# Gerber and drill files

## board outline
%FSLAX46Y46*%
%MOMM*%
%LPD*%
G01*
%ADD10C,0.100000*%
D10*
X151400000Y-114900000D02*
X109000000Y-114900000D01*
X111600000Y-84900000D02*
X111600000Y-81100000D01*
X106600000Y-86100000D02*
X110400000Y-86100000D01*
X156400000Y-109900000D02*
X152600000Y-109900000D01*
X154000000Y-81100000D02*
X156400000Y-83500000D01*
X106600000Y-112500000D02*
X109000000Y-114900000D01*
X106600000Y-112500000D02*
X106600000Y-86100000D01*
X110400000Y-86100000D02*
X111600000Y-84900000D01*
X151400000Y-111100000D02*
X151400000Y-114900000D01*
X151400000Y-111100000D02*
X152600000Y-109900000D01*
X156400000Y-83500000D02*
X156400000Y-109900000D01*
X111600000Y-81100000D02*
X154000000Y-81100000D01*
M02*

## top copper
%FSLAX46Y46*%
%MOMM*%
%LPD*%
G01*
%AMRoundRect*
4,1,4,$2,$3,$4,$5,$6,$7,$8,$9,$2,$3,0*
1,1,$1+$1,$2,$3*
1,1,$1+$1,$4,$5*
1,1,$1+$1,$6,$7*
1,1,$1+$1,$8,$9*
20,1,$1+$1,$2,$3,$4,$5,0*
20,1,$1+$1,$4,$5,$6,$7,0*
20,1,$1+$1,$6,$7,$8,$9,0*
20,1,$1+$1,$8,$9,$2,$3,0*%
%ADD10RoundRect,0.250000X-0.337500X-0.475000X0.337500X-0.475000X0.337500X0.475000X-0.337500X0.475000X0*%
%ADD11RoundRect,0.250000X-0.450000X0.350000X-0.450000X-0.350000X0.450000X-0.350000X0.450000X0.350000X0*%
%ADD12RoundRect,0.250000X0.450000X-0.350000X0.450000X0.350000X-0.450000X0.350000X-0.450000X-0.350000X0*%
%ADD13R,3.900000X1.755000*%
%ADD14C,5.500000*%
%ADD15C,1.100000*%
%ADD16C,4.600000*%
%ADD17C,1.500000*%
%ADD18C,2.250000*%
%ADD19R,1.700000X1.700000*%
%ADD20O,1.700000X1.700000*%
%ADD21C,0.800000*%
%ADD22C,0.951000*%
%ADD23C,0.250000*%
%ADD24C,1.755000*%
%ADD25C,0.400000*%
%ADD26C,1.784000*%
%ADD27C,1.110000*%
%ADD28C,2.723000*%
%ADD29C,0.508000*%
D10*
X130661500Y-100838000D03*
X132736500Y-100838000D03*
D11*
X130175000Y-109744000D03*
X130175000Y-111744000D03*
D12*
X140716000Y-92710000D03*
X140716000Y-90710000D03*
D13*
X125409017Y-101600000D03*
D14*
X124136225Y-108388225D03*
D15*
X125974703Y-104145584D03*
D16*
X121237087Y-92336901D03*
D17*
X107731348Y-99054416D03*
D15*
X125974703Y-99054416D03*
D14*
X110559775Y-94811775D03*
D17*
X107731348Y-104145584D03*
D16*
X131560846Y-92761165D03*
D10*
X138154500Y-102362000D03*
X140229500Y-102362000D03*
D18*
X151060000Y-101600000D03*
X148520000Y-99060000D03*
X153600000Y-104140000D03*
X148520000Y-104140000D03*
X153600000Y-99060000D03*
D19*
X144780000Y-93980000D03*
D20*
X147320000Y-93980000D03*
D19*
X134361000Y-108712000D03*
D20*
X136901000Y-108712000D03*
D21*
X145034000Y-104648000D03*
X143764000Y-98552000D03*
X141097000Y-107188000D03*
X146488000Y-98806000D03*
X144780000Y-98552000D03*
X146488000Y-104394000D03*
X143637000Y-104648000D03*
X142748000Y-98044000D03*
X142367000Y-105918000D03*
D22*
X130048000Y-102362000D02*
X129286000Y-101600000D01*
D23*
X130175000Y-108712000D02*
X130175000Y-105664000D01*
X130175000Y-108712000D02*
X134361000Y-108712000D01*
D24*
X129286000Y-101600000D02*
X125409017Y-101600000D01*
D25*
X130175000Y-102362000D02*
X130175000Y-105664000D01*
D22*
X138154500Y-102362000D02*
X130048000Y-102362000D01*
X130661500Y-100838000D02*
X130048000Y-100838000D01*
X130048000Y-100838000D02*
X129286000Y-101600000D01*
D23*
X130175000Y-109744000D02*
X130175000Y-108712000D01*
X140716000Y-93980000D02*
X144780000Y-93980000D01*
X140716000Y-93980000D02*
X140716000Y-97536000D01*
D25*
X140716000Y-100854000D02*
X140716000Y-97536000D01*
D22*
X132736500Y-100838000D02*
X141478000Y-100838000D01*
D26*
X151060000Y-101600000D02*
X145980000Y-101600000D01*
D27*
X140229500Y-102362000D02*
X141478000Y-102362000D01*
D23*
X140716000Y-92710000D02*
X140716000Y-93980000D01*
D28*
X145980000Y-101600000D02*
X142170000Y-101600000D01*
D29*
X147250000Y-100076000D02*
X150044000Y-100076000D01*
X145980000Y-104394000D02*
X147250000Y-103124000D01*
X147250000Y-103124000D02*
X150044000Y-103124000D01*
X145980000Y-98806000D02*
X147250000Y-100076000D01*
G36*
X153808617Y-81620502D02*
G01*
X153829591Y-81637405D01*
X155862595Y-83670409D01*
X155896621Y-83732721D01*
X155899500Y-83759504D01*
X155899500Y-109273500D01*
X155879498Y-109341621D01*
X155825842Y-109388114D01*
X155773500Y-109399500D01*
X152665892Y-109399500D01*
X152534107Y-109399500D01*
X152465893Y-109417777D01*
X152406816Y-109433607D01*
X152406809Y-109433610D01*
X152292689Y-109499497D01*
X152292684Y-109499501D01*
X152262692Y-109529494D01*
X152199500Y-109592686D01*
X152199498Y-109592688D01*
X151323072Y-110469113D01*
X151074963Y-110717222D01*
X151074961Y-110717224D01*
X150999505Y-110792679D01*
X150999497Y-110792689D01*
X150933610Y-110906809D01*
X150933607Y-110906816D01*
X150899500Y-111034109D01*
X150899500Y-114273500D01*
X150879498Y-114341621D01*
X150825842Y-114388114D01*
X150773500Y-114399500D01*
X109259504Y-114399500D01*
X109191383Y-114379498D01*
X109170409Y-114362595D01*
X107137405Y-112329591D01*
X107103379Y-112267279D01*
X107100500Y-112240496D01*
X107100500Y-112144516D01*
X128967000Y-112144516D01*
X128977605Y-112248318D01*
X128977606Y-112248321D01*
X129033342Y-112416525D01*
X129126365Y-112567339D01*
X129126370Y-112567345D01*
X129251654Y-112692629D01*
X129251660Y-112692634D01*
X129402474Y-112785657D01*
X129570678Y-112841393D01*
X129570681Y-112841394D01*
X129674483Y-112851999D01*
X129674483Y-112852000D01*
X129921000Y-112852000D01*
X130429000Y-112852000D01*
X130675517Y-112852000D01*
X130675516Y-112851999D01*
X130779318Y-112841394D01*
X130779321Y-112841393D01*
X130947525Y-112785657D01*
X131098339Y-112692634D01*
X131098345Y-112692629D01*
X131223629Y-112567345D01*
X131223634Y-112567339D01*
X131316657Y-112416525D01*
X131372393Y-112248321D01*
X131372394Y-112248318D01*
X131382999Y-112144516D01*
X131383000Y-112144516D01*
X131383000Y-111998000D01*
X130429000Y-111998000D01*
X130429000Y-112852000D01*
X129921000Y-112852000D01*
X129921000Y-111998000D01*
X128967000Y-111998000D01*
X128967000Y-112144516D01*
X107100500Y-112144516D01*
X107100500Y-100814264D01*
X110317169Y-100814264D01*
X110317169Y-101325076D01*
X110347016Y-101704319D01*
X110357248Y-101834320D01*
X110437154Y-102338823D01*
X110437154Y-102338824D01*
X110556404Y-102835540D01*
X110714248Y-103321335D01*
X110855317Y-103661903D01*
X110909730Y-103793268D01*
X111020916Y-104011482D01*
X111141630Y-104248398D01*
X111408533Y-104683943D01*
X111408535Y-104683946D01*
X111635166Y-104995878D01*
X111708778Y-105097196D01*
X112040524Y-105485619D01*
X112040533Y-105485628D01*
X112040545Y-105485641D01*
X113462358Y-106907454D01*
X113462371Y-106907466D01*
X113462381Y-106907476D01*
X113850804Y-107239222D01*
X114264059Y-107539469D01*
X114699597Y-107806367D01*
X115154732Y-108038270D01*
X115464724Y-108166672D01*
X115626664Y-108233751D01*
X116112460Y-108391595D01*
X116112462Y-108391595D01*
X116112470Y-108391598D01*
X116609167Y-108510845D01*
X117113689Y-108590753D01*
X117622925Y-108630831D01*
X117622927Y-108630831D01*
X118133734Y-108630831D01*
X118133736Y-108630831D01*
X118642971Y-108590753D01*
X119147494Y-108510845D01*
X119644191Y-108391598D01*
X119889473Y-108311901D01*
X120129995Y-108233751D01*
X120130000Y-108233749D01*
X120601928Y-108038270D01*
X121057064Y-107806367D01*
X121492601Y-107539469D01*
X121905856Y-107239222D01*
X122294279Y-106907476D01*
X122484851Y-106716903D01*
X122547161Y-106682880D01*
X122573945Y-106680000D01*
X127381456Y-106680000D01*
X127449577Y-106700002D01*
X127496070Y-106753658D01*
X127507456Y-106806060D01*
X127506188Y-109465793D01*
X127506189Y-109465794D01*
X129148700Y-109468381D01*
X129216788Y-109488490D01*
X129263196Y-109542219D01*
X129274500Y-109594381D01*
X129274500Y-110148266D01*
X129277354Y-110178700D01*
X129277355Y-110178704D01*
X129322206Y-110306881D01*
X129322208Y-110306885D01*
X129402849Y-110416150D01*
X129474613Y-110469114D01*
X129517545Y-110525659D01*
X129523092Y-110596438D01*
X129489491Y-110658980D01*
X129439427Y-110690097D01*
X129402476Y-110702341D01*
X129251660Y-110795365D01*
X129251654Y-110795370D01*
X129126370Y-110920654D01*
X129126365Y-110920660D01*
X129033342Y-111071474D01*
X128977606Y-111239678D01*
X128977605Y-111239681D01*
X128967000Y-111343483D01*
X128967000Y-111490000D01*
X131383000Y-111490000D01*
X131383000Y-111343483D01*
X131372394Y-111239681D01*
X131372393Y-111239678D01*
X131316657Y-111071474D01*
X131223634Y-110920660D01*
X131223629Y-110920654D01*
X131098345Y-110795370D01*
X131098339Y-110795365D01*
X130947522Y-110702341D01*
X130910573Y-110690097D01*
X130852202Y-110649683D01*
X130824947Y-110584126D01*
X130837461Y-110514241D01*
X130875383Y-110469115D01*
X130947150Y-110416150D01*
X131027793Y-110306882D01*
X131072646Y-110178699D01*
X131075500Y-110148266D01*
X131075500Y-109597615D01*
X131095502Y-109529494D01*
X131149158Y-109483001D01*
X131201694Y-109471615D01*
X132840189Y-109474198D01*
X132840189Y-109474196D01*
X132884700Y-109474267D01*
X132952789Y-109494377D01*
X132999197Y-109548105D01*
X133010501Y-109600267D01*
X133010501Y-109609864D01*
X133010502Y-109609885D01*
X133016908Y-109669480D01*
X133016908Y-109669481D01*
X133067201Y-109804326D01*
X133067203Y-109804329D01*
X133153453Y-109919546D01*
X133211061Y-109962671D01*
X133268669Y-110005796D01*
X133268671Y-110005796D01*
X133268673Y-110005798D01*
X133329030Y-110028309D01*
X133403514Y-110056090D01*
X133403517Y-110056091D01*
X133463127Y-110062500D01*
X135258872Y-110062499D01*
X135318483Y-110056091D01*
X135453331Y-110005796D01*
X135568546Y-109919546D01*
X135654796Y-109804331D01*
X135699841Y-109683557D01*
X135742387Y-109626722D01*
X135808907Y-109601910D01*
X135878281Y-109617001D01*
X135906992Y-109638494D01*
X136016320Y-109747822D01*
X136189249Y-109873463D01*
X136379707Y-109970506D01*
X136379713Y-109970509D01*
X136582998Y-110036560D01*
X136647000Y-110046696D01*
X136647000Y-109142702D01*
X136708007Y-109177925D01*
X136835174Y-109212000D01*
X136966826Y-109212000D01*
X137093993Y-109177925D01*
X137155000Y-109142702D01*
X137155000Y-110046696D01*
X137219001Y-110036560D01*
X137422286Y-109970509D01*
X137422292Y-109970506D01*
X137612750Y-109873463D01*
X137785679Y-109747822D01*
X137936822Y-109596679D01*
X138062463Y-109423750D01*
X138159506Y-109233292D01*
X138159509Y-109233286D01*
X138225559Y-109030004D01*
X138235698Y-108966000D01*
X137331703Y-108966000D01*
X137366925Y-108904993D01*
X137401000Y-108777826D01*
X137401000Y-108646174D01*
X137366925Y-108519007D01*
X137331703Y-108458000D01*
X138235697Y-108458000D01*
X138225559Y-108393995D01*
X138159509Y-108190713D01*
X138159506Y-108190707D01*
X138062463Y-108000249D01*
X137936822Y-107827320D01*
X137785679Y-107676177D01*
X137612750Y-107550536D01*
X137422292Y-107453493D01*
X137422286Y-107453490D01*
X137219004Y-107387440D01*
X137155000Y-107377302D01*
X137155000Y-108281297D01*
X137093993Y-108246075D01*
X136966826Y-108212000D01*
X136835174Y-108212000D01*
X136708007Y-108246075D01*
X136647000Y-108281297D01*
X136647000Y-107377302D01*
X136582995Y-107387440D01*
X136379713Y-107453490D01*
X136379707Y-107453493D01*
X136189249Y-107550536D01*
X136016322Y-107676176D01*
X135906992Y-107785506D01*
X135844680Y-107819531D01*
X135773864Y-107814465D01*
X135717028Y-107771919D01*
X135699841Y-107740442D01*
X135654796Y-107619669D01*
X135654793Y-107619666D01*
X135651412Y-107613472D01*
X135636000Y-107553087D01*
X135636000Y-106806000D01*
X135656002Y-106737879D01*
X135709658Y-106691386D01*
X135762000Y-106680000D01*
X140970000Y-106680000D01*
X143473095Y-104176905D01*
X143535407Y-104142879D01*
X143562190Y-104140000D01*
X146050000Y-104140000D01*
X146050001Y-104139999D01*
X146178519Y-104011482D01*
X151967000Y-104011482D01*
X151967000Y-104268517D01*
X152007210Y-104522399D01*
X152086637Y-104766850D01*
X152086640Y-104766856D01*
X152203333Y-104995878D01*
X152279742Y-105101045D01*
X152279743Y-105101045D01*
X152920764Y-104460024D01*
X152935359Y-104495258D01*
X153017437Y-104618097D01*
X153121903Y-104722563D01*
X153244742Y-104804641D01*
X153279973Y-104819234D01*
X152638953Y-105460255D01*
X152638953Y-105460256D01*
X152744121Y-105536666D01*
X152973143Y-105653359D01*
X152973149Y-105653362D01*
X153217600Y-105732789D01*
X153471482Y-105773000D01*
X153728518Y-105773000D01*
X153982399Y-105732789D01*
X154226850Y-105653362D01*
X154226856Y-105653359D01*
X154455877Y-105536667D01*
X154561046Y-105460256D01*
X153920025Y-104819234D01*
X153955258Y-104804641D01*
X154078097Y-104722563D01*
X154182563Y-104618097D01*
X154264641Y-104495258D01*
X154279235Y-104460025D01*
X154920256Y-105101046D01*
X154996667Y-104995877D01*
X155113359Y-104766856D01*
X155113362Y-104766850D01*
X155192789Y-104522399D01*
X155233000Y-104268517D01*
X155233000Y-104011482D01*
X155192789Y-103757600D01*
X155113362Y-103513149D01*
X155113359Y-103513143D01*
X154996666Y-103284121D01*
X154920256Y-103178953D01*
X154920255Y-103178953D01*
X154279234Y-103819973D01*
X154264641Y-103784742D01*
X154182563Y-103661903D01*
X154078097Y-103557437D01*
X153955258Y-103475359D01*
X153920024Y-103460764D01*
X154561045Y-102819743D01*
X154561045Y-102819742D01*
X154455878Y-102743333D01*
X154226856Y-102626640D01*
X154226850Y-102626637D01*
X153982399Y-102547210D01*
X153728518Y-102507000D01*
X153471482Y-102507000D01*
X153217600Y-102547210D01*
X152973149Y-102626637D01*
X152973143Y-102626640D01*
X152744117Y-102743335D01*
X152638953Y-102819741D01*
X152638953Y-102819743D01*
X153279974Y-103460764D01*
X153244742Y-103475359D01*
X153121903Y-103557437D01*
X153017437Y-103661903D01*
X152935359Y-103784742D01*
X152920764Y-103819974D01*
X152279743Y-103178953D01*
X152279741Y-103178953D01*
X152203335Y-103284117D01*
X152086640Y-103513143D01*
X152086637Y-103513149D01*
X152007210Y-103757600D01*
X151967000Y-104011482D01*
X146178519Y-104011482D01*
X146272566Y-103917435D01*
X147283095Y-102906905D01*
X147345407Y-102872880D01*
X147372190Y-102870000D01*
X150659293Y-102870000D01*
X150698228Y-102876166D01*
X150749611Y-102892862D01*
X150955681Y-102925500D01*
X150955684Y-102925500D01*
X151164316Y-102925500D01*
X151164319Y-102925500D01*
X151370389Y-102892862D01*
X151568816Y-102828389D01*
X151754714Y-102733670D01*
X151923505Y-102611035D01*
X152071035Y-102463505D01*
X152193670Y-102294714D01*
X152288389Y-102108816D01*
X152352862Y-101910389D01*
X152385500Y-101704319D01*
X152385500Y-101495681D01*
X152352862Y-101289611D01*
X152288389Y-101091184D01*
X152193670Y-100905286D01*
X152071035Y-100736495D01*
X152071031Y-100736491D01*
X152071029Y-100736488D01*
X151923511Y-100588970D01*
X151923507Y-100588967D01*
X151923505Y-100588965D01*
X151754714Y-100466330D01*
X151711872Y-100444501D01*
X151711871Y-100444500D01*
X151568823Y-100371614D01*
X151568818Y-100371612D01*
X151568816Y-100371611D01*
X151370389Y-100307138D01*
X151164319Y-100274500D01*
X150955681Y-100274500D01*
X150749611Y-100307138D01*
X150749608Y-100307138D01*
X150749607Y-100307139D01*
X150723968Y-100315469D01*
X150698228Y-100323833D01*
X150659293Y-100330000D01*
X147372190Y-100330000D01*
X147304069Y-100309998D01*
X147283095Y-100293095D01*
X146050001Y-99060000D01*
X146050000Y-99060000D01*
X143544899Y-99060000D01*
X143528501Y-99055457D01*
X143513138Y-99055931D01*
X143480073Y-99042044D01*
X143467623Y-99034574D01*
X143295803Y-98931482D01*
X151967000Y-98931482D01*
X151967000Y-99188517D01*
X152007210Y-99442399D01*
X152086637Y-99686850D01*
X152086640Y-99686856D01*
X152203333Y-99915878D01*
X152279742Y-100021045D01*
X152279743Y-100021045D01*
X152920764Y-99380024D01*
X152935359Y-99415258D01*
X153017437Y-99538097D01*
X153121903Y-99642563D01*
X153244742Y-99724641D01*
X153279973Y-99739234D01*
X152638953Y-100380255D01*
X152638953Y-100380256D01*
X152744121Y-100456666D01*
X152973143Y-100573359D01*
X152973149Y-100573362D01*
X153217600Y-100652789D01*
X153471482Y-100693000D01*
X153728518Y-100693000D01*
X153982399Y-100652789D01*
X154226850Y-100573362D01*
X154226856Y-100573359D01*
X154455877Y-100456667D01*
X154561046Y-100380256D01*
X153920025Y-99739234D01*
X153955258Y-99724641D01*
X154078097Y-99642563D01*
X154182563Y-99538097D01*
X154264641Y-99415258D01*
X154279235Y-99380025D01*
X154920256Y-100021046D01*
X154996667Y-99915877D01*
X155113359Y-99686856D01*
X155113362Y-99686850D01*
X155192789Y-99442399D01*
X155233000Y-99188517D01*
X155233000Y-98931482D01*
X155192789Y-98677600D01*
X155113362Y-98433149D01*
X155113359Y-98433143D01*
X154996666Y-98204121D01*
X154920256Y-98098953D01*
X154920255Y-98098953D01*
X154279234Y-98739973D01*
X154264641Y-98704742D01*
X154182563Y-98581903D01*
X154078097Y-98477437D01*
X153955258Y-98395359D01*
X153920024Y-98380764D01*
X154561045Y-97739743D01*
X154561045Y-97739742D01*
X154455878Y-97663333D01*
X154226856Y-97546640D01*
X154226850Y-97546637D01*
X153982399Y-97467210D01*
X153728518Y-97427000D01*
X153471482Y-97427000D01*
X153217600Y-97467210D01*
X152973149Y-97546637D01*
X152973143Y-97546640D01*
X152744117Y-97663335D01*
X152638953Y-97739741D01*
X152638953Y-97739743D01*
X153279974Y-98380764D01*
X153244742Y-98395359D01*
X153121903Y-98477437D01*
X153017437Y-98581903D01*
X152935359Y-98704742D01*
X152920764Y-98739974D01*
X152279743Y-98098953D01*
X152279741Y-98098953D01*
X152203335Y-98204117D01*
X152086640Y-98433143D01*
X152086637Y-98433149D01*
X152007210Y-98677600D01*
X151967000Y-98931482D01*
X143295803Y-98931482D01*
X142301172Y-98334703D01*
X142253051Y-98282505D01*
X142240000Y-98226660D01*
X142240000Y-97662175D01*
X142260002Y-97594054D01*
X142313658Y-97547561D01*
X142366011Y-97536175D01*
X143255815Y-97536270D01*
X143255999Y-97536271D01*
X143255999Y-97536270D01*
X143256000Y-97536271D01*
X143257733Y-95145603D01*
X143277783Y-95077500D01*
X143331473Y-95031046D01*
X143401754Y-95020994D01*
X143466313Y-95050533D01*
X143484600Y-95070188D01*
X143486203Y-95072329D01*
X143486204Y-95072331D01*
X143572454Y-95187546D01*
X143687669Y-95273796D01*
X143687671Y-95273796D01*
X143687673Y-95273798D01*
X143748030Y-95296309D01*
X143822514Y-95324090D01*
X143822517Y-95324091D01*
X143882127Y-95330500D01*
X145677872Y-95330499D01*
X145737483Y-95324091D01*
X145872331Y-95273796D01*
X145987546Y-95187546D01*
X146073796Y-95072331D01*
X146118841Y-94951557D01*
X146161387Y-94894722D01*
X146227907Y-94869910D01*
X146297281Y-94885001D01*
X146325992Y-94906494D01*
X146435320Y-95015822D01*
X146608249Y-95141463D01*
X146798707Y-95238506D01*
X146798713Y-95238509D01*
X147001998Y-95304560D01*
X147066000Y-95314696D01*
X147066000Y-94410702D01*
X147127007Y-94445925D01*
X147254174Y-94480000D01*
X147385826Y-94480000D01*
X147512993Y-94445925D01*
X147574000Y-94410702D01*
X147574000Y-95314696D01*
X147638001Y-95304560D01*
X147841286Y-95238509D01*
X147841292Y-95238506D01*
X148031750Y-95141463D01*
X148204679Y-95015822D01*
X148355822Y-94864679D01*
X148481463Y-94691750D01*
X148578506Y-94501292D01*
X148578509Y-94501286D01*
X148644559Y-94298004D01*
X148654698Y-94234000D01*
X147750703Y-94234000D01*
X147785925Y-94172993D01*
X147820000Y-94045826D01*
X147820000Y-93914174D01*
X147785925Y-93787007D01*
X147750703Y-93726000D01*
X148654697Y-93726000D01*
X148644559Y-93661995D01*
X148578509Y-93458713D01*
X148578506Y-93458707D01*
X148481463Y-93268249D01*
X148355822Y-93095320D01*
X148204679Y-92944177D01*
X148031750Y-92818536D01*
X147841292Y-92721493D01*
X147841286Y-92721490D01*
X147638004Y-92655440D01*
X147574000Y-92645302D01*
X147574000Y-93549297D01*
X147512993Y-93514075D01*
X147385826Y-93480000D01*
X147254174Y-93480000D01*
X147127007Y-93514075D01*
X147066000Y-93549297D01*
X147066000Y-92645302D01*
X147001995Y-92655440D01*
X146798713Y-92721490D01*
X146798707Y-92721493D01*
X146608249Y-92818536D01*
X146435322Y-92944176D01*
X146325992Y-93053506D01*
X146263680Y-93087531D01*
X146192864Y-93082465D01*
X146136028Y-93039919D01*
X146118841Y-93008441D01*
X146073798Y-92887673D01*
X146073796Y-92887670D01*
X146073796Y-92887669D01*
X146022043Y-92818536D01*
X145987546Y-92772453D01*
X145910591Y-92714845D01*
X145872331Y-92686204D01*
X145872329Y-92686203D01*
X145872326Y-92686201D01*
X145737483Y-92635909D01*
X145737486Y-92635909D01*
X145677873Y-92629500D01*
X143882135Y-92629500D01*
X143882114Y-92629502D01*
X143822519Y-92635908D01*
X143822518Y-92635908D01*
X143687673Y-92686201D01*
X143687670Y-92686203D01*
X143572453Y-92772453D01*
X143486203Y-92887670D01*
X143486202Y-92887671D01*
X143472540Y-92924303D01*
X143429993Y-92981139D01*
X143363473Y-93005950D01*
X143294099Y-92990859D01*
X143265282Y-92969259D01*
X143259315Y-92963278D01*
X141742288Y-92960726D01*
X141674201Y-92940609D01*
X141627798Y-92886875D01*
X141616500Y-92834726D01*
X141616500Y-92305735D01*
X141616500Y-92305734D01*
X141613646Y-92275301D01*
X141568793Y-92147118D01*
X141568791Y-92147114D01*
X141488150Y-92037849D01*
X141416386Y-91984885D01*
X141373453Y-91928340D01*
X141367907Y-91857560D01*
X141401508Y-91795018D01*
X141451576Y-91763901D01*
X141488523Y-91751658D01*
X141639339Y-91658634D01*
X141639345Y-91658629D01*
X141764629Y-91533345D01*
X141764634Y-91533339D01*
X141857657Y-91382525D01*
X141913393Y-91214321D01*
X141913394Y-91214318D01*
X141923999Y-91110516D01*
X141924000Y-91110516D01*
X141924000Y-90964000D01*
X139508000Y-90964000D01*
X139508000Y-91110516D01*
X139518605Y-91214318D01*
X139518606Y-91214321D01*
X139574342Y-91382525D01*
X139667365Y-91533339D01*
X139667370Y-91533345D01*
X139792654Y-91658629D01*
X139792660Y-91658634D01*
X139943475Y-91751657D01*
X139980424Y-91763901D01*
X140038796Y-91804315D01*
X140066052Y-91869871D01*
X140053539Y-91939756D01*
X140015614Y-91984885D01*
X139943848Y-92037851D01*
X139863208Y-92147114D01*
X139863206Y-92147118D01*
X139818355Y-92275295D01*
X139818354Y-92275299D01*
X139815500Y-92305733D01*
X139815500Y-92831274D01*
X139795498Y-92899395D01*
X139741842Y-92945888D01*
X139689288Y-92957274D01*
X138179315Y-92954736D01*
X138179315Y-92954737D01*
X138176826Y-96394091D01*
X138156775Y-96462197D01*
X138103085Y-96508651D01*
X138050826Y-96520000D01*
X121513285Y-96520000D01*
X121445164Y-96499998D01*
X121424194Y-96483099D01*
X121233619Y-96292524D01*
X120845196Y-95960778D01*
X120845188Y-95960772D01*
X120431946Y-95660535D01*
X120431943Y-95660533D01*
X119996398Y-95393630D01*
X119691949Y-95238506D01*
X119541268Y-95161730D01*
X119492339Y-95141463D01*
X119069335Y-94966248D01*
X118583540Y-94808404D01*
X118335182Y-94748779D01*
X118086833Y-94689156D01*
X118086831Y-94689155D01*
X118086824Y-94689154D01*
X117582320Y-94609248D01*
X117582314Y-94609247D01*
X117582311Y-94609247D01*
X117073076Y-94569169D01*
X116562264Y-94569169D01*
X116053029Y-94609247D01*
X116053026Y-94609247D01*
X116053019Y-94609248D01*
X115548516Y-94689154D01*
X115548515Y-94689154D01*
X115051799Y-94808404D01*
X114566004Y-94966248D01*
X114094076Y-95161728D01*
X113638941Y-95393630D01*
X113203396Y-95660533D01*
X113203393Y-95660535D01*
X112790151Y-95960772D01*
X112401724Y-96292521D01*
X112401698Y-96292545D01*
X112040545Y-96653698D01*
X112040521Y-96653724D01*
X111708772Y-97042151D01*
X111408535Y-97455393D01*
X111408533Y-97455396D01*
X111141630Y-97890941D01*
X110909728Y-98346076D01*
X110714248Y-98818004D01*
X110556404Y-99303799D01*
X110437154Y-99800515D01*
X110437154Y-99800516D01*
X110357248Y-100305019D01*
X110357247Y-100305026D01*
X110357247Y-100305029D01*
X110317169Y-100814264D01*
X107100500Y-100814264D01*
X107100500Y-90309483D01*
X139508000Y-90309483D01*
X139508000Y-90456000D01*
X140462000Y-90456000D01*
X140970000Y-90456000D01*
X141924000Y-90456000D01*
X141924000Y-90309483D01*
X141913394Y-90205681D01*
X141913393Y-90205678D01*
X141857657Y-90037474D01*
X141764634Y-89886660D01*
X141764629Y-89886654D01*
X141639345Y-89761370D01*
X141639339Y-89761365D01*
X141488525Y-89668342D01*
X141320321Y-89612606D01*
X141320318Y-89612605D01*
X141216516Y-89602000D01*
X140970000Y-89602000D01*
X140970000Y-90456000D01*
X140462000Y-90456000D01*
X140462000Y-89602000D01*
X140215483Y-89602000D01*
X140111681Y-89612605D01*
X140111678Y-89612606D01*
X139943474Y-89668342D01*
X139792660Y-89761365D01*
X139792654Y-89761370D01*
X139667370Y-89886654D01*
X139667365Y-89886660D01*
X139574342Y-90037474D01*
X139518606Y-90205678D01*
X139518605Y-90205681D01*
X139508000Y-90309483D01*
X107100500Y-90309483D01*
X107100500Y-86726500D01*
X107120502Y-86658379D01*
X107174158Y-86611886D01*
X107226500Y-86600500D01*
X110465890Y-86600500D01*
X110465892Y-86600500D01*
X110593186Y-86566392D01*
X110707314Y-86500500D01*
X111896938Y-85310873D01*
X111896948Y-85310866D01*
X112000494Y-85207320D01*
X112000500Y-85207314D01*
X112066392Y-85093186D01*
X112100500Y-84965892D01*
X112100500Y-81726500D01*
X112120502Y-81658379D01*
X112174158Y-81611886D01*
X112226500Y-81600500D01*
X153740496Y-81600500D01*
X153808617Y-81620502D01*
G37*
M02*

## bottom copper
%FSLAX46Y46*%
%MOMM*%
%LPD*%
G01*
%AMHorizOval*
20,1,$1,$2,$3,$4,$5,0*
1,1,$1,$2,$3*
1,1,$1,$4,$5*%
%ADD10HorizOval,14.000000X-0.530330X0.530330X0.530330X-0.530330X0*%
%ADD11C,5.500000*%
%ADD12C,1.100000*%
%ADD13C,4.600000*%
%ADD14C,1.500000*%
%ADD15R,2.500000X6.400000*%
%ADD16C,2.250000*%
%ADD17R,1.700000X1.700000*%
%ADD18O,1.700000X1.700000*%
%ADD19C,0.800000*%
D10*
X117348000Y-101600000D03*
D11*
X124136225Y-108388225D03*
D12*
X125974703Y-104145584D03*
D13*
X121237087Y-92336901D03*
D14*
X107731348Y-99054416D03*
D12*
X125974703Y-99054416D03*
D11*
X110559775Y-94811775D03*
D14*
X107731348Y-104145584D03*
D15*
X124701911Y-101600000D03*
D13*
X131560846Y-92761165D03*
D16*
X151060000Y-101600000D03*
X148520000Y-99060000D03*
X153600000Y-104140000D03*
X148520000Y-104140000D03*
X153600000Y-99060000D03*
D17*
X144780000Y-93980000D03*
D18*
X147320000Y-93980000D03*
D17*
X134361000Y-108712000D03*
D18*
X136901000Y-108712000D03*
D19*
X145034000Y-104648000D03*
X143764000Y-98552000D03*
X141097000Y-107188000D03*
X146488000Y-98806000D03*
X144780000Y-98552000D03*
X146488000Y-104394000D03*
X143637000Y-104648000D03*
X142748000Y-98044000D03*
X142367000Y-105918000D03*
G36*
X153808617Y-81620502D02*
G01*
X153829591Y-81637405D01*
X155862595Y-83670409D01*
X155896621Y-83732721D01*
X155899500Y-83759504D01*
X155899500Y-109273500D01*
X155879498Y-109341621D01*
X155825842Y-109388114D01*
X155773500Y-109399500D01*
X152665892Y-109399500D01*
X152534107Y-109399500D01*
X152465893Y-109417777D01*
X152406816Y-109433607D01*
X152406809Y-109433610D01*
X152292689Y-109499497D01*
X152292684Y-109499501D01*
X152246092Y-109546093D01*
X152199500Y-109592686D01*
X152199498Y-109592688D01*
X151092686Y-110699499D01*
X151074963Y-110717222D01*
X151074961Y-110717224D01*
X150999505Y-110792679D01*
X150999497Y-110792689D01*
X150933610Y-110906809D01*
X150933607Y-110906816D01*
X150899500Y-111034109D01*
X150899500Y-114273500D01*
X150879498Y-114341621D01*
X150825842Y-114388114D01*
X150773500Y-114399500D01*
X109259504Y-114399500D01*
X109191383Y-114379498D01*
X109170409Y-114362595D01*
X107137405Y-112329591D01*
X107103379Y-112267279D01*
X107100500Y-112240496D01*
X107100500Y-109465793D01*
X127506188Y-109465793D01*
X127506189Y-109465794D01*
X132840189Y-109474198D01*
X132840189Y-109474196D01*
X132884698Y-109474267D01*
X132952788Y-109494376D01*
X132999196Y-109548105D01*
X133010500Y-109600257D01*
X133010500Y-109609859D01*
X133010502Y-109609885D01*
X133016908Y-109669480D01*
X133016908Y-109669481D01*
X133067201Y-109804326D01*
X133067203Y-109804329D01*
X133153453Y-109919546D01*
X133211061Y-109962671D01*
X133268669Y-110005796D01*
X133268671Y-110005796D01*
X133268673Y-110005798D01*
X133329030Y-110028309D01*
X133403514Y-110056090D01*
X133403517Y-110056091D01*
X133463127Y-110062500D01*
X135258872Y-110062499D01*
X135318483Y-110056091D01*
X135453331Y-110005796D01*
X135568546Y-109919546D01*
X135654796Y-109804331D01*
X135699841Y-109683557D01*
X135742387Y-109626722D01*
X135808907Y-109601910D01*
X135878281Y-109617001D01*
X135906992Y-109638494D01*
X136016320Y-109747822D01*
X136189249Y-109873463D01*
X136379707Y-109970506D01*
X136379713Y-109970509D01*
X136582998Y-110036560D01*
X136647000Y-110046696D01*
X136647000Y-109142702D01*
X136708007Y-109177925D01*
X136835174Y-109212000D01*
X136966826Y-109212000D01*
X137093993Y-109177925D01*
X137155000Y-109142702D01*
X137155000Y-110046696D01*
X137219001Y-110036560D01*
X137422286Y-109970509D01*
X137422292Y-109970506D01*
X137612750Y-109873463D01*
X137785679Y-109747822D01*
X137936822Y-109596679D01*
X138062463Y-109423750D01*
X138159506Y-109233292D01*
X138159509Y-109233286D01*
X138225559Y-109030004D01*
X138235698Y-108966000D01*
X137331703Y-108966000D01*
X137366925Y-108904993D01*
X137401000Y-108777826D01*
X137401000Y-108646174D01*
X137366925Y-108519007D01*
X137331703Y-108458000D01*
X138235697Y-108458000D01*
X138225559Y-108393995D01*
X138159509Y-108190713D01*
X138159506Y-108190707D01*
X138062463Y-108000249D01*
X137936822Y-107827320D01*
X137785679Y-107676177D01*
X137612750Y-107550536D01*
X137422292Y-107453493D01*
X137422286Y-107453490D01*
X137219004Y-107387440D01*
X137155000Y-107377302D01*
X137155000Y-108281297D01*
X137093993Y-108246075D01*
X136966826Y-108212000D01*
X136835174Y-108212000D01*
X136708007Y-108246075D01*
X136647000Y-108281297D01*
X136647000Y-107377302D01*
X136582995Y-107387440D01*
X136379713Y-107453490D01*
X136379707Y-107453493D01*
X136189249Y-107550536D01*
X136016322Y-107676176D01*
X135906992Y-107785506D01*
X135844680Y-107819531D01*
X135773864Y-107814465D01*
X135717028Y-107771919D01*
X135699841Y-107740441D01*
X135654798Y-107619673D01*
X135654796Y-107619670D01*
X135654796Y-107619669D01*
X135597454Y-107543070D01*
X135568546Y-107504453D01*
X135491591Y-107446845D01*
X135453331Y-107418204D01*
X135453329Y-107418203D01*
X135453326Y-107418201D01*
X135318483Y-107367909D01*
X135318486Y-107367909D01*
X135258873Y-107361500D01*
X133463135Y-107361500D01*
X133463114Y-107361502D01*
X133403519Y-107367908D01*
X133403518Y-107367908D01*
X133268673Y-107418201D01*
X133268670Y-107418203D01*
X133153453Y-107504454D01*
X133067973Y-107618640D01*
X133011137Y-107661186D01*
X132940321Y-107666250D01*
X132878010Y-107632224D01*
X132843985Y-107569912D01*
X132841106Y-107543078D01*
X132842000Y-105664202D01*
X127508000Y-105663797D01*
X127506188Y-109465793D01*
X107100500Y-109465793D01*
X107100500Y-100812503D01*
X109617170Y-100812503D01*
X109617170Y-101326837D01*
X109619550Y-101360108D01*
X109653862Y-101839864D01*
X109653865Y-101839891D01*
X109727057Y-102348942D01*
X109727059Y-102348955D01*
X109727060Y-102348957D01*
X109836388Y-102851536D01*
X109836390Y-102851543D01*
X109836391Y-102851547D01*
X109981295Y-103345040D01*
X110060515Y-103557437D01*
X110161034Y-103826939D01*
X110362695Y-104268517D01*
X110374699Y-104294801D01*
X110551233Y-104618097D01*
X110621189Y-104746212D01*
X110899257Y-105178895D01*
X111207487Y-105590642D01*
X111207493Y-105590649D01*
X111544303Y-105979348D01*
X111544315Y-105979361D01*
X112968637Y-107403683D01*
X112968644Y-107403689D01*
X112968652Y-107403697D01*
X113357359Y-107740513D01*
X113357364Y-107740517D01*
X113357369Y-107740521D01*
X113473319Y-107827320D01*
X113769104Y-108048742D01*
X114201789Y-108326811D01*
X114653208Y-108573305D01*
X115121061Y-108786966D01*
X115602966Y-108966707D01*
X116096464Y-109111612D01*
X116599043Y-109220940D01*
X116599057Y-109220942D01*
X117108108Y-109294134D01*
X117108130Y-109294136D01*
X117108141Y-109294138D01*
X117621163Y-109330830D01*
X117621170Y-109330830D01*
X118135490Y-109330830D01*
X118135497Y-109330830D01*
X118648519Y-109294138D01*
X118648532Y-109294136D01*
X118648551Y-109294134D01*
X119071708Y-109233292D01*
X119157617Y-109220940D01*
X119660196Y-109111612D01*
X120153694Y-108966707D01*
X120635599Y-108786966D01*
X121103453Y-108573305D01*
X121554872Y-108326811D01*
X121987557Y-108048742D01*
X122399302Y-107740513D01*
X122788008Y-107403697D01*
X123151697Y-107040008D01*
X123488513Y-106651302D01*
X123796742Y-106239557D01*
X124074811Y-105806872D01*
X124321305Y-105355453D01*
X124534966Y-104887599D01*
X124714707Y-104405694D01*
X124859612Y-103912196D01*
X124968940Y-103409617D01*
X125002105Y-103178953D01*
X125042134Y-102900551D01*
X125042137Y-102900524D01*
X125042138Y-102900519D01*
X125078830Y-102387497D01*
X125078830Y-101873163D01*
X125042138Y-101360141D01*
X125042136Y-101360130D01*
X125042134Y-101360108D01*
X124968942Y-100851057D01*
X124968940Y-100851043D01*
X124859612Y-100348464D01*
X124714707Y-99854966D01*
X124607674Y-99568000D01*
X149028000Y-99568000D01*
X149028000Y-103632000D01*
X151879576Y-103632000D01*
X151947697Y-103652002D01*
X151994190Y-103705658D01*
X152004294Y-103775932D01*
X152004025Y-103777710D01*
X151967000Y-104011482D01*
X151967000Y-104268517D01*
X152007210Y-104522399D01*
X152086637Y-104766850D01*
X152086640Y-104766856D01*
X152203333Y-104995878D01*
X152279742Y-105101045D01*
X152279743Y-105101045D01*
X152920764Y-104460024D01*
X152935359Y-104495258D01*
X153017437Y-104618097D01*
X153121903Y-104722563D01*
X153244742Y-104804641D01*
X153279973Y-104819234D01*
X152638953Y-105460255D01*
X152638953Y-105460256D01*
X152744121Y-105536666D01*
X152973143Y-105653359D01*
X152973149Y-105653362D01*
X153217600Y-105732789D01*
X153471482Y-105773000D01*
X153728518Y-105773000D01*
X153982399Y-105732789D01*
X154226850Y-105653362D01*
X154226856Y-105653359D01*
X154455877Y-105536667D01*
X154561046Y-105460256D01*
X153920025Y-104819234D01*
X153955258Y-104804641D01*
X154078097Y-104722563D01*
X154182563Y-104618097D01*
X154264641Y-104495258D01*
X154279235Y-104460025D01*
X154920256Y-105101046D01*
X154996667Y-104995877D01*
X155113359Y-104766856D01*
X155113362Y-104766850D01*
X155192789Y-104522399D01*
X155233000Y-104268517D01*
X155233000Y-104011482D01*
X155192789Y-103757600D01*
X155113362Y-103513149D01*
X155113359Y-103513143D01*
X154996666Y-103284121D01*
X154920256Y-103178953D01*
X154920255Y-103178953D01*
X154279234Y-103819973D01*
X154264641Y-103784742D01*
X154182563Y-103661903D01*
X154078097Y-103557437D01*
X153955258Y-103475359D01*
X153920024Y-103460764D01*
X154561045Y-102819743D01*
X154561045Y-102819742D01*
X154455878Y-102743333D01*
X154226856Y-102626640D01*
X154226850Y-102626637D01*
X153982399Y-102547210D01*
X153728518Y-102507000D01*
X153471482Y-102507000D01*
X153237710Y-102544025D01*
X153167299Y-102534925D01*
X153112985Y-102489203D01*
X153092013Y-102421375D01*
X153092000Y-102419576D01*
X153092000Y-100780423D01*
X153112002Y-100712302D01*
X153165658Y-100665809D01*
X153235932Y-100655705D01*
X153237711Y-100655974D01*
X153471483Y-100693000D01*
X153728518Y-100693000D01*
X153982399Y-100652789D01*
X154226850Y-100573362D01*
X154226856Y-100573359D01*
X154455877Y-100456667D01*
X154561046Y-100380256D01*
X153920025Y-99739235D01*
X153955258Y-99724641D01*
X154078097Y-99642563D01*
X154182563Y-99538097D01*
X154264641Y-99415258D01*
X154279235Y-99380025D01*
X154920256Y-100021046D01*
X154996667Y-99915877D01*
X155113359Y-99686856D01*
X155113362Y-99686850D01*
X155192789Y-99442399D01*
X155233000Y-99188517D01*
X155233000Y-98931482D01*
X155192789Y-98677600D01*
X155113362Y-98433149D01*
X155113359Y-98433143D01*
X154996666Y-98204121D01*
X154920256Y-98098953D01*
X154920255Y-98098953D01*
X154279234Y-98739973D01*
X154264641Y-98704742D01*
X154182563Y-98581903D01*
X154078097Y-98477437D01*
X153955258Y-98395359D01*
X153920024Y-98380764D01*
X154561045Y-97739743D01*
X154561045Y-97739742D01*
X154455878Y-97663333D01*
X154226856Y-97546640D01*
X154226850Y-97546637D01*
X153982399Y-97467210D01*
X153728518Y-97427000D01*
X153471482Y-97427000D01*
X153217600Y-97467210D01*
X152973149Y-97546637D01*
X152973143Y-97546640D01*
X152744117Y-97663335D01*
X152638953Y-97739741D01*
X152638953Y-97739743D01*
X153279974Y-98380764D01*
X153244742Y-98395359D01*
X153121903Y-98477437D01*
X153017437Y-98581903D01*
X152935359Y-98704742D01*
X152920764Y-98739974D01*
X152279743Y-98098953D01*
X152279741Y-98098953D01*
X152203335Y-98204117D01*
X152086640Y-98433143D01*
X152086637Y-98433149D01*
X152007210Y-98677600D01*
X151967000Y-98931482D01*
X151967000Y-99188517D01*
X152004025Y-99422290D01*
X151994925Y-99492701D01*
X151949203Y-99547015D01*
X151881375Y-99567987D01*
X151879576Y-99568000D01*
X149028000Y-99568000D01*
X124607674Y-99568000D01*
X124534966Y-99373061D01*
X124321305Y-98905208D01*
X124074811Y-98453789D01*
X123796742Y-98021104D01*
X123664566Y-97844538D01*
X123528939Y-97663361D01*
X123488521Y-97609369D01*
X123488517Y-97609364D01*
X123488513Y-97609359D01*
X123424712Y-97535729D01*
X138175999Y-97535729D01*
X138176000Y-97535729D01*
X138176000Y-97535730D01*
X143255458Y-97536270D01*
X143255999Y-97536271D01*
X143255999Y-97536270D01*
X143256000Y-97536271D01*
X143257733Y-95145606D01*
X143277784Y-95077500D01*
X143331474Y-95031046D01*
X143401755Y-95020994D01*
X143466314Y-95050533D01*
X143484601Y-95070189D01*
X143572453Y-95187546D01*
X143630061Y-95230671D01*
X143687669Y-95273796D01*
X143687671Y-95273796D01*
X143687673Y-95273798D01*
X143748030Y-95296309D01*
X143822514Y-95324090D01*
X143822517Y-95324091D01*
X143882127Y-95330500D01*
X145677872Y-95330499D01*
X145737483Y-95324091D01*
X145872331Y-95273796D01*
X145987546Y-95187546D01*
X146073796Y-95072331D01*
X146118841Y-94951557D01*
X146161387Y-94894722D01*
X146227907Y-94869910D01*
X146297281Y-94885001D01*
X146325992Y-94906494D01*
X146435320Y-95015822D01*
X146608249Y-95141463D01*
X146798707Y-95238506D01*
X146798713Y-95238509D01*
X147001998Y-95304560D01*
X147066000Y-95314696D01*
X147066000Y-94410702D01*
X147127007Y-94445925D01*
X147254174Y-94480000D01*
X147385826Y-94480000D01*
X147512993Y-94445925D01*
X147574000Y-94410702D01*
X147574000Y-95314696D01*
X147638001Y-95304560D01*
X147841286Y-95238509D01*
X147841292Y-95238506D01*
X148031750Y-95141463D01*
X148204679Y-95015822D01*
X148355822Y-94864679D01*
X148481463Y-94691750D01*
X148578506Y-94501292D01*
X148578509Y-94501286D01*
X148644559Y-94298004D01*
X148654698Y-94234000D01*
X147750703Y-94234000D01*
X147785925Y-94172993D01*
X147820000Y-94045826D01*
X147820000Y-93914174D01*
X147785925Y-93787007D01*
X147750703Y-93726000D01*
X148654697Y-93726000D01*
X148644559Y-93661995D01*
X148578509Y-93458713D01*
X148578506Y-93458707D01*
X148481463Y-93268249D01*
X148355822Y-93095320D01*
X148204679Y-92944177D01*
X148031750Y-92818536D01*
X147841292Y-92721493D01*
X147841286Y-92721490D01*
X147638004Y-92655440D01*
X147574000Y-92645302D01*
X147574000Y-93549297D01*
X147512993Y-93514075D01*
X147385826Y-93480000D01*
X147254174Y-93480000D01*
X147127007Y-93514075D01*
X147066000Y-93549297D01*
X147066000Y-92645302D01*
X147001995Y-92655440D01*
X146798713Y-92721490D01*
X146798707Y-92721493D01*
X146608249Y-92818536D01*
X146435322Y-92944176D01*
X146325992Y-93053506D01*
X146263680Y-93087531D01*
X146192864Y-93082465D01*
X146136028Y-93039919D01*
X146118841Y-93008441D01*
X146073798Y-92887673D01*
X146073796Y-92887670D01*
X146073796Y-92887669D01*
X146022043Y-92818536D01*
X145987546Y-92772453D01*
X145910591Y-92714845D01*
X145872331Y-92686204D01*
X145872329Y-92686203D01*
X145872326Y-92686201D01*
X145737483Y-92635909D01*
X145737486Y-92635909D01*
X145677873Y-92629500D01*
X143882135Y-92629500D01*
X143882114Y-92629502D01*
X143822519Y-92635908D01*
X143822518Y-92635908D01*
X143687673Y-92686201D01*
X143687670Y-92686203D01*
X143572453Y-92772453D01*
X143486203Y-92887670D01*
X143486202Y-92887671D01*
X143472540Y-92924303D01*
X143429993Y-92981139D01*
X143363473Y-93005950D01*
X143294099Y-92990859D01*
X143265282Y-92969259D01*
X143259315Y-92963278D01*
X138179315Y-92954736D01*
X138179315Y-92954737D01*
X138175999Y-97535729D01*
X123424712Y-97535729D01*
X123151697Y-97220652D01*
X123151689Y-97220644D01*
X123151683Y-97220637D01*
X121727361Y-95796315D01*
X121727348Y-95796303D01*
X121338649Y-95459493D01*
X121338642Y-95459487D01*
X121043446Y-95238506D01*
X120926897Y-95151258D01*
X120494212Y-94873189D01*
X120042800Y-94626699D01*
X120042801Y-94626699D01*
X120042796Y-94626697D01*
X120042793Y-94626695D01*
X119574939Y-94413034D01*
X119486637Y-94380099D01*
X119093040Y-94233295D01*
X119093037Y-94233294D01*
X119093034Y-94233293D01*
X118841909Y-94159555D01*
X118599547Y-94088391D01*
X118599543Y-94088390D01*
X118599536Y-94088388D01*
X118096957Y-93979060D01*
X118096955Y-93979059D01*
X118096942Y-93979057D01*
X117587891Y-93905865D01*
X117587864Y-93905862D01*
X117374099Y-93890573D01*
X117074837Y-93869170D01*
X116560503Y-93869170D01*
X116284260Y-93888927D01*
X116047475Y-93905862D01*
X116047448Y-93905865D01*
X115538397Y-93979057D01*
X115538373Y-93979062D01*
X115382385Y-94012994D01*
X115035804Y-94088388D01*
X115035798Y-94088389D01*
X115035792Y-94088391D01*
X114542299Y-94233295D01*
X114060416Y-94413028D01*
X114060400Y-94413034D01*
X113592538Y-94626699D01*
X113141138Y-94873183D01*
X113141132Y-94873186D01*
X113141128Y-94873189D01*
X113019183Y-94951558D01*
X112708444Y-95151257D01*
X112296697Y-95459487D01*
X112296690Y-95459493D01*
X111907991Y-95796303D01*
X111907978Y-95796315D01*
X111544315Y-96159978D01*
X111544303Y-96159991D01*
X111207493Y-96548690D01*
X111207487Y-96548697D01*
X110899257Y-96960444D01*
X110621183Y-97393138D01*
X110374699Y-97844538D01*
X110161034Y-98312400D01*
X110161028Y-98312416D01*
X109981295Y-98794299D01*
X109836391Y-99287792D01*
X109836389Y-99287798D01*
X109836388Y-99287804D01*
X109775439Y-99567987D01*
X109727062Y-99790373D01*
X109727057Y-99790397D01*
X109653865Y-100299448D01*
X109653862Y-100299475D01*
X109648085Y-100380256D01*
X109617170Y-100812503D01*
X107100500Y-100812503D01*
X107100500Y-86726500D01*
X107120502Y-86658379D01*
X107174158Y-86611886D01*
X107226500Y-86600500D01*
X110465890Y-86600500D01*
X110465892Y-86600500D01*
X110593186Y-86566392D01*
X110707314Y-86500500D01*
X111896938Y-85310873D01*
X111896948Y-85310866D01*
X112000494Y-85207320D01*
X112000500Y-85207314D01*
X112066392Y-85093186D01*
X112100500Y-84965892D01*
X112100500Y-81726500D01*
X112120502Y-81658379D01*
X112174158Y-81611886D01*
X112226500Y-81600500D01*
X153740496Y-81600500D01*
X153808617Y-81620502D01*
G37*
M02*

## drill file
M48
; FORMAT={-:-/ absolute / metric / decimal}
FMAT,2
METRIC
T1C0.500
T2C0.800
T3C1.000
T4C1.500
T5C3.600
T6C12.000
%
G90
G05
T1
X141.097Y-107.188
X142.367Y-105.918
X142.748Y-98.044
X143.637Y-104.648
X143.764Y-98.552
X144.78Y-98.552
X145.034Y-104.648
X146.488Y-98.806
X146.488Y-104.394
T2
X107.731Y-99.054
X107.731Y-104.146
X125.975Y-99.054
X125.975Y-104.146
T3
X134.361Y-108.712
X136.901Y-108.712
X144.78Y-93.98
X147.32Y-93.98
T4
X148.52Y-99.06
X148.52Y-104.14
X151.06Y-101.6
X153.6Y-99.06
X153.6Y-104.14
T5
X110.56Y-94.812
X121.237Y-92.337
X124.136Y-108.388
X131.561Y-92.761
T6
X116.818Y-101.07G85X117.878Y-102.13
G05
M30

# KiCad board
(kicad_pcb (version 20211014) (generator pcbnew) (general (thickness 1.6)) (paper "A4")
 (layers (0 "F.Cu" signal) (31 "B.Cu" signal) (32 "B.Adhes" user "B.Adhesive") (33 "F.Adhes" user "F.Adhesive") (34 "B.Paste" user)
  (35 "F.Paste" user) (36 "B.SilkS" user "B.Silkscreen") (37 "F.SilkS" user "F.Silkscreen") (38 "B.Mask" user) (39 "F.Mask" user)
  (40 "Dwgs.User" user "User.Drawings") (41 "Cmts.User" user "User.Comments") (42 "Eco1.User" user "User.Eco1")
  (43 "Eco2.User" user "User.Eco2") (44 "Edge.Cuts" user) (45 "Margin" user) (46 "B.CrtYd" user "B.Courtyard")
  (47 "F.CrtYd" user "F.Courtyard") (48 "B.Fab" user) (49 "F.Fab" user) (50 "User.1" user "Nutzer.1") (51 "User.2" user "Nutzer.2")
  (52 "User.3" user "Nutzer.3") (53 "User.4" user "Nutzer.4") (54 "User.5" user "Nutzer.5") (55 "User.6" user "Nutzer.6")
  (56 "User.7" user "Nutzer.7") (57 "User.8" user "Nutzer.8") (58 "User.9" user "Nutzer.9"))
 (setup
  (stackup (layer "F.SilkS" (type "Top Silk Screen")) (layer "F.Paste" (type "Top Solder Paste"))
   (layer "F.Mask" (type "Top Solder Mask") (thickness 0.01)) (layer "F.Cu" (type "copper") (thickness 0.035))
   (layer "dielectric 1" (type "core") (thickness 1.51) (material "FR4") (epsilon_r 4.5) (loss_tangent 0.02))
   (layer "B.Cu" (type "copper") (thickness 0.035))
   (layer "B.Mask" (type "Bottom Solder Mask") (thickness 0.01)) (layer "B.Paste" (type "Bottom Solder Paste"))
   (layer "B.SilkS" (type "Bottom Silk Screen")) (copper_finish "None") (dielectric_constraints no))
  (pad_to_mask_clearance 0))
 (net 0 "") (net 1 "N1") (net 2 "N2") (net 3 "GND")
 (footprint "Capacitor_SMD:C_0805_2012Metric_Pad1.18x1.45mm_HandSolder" (layer "F.Cu") (at 131.699 100.838)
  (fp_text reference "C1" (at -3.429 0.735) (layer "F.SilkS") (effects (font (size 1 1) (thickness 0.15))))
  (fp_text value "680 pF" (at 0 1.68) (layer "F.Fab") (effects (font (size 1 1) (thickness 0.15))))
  (pad "1" smd roundrect (at -1.0375 0) (size 1.175 1.45) (layers "F.Cu" "F.Paste" "F.Mask") (roundrect_rratio 0.212766) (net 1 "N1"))
  (pad "2" smd roundrect (at 1.0375 0) (size 1.175 1.45) (layers "F.Cu" "F.Paste" "F.Mask") (roundrect_rratio 0.212766) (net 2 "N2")))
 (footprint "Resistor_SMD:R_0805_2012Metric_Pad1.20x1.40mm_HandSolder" (layer "F.Cu") (at 130.175 110.744 -90)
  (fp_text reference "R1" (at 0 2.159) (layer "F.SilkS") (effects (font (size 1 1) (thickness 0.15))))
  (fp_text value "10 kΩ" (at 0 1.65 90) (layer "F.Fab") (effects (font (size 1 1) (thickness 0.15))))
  (pad "1" smd roundrect (at -1 0 270) (size 1.2 1.4) (layers "F.Cu" "F.Paste" "F.Mask") (roundrect_rratio 0.208333) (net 1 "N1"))
  (pad "2" smd roundrect (at 1 0 270) (size 1.2 1.4) (layers "F.Cu" "F.Paste" "F.Mask") (roundrect_rratio 0.208333) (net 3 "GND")))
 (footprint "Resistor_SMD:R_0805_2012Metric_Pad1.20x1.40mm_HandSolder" (layer "F.Cu") (at 140.716 91.71 90)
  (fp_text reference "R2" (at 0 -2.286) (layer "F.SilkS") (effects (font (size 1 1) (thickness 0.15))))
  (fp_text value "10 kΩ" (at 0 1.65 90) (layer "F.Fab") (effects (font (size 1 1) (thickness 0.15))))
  (pad "1" smd roundrect (at -1 0 90) (size 1.2 1.4) (layers "F.Cu" "F.Paste" "F.Mask") (roundrect_rratio 0.208333) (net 2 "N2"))
  (pad "2" smd roundrect (at 1 0 90) (size 1.2 1.4) (layers "F.Cu" "F.Paste" "F.Mask") (roundrect_rratio 0.208333) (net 3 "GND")))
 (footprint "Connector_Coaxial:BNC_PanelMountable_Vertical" (layer "F.Cu") (at 117.348 101.6 45)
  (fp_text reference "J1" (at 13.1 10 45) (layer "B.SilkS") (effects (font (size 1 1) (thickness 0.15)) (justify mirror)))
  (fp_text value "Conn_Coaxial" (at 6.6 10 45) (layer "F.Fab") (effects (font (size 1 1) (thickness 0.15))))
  (pad "" np_thru_hole oval (at 0 0 45) (size 14 15.5) (drill oval 12 13.5) (layers *.Mask "B.Cu"))
  (pad "1" connect rect (at 5.7 5.7 90) (size 1.755 3.9) (layers "F.Cu" "F.Mask") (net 1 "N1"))
  (pad "2" thru_hole circle (at 0 9.6 45) (size 5.5 5.5) (drill 3.6) (layers *.Cu *.Mask) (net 3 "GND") (zone_connect 2))
  (pad "2" thru_hole circle (at 4.3 7.9 45) (size 1.1 1.1) (drill 0.8) (layers *.Cu *.Mask) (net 3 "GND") (solder_mask_margin 0.3)
   (zone_connect 2))
  (pad "2" thru_hole circle (at 9.3 -3.8 45) (size 4.6 4.6) (drill 3.6) (layers *.Cu *.Mask) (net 3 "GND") (zone_connect 2))
  (pad "2" thru_hole circle (at -5 -8.6 45) (size 1.5 1.5) (drill 0.8) (layers *.Cu *.Mask) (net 3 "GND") (zone_connect 2))
  (pad "2" thru_hole circle (at 7.9 4.3 45) (size 1.1 1.1) (drill 0.8) (layers *.Cu *.Mask) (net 3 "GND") (solder_mask_margin 0.3)
   (zone_connect 2))
  (pad "2" thru_hole circle (at 0 -9.6 45) (size 5.5 5.5) (drill 3.6) (layers *.Cu *.Mask) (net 3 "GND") (zone_connect 2))
  (pad "2" thru_hole circle (at -8.6 -5 45) (size 1.5 1.5) (drill 0.8) (layers *.Cu *.Mask) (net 3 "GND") (zone_connect 2))
  (pad "2" connect rect (at 5.2 5.2) (size 2.5 6.4) (layers "B.Cu" "B.Mask") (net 3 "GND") (zone_connect 2))
  (pad "2" thru_hole circle (at 16.3 3.8 45) (size 4.6 4.6) (drill 3.6) (layers *.Cu *.Mask) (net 3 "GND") (zone_connect 2)))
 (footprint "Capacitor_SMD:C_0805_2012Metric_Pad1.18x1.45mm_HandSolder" (layer "F.Cu") (at 139.192 102.362)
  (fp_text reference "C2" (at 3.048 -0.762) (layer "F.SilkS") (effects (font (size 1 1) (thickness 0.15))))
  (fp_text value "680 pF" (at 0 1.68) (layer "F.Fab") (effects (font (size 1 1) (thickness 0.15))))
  (pad "1" smd roundrect (at -1.0375 0) (size 1.175 1.45) (layers "F.Cu" "F.Paste" "F.Mask") (roundrect_rratio 0.212766) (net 1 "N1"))
  (pad "2" smd roundrect (at 1.0375 0) (size 1.175 1.45) (layers "F.Cu" "F.Paste" "F.Mask") (roundrect_rratio 0.212766) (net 2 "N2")))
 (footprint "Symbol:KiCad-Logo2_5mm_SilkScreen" (layer "B.Cu") (at 131.5 98 -90)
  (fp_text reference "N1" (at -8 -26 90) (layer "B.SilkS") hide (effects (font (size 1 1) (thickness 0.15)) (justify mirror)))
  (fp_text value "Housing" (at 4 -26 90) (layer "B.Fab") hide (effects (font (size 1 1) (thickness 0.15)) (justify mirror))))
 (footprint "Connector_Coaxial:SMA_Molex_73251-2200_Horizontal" (layer "B.Cu") (at 151.06 101.6 90)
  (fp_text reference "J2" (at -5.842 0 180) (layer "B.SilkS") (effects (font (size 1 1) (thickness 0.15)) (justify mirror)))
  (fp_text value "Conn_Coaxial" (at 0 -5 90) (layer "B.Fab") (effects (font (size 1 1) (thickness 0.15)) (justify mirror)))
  (pad "1" thru_hole circle (at 0 0 90) (size 2.25 2.25) (drill 1.5) (layers *.Cu *.Mask) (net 2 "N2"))
  (pad "2" thru_hole circle (at 2.54 -2.54) (size 2.25 2.25) (drill 1.5) (layers *.Cu *.Mask) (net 3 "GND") (zone_connect 2))
  (pad "2" thru_hole circle (at -2.54 2.54 90) (size 2.25 2.25) (drill 1.5) (layers *.Cu *.Mask) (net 3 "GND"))
  (pad "2" thru_hole circle (at -2.54 -2.54 90) (size 2.25 2.25) (drill 1.5) (layers *.Cu *.Mask) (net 3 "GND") (zone_connect 2))
  (pad "2" thru_hole circle (at 2.54 2.54 90) (size 2.25 2.25) (drill 1.5) (layers *.Cu *.Mask) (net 3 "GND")))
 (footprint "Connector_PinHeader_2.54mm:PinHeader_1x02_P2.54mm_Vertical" (layer "B.Cu") (at 144.78 93.98 -90)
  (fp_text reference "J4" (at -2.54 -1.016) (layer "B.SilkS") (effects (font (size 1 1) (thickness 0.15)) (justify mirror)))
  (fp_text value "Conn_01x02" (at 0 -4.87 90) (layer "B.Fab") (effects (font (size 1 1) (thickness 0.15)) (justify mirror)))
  (pad "1" thru_hole rect (at 0 0 270) (size 1.7 1.7) (drill 1) (layers *.Cu *.Mask) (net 2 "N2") (clearance 0.5))
  (pad "2" thru_hole oval (at 0 -2.54 270) (size 1.7 1.7) (drill 1) (layers *.Cu *.Mask) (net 3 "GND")))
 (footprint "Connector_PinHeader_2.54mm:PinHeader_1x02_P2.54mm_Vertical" (layer "B.Cu") (at 134.361 108.712 -90)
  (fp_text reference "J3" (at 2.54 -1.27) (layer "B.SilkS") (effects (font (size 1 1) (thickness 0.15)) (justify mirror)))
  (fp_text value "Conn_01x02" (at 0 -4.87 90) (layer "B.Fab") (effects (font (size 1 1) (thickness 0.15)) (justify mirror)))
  (pad "1" thru_hole rect (at 0 0 270) (size 1.7 1.7) (drill 1) (layers *.Cu *.Mask) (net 1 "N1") (clearance 0.5))
  (pad "2" thru_hole oval (at 0 -2.54 270) (size 1.7 1.7) (drill 1) (layers *.Cu *.Mask) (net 3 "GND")))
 (gr_line (start 151.4 114.9) (end 109 114.9) (layer "Edge.Cuts") (width 0.1))
 (gr_line (start 111.6 84.9) (end 111.6 81.1) (layer "Edge.Cuts") (width 0.1))
 (gr_line (start 106.6 86.1) (end 110.4 86.1) (layer "Edge.Cuts") (width 0.1))
 (gr_line (start 156.4 109.9) (end 152.6 109.9) (layer "Edge.Cuts") (width 0.1))
 (gr_line (start 154 81.1) (end 156.4 83.5) (layer "Edge.Cuts") (width 0.1))
 (gr_line (start 106.6 112.5) (end 109 114.9) (layer "Edge.Cuts") (width 0.1))
 (gr_line (start 106.6 112.5) (end 106.6 86.1) (layer "Edge.Cuts") (width 0.1))
 (gr_line (start 110.4 86.1) (end 111.6 84.9) (layer "Edge.Cuts") (width 0.1))
 (gr_line (start 151.4 111.1) (end 151.4 114.9) (layer "Edge.Cuts") (width 0.1))
 (gr_line (start 151.4 111.1) (end 152.6 109.9) (layer "Edge.Cuts") (width 0.1))
 (gr_line (start 156.4 83.5) (end 156.4 109.9) (layer "Edge.Cuts") (width 0.1))
 (gr_line (start 111.6 81.1) (end 154 81.1) (layer "Edge.Cuts") (width 0.1))
 (segment (start 130.048 102.362) (end 129.286 101.6) (width 0.951) (layer "F.Cu") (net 1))
 (segment (start 130.175 108.712) (end 130.175 105.664) (width 0.25) (layer "F.Cu") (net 1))
 (segment (start 130.175 108.712) (end 134.361 108.712) (width 0.25) (layer "F.Cu") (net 1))
 (segment (start 129.286 101.6) (end 125.409017 101.6) (width 1.755) (layer "F.Cu") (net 1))
 (segment (start 130.175 102.362) (end 130.175 105.664) (width 0.4) (layer "F.Cu") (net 1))
 (segment (start 138.1545 102.362) (end 130.048 102.362) (width 0.951) (layer "F.Cu") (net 1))
 (segment (start 130.6615 100.838) (end 130.048 100.838) (width 0.951) (layer "F.Cu") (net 1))
 (segment (start 130.048 100.838) (end 129.286 101.6) (width 0.951) (layer "F.Cu") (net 1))
 (segment (start 130.175 109.744) (end 130.175 108.712) (width 0.25) (layer "F.Cu") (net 1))
 (segment (start 140.716 93.98) (end 144.78 93.98) (width 0.25) (layer "F.Cu") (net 2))
 (segment (start 140.716 93.98) (end 140.716 97.536) (width 0.25) (layer "F.Cu") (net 2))
 (segment (start 140.716 100.854) (end 140.716 97.536) (width 0.4) (layer "F.Cu") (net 2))
 (segment (start 132.7365 100.838) (end 141.478 100.838) (width 0.951) (layer "F.Cu") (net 2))
 (segment (start 151.06 101.6) (end 145.98 101.6) (width 1.784) (layer "F.Cu") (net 2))
 (segment (start 140.2295 102.362) (end 141.478 102.362) (width 1.11) (layer "F.Cu") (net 2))
 (segment (start 140.716 92.71) (end 140.716 93.98) (width 0.25) (layer "F.Cu") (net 2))
 (segment (start 145.98 101.6) (end 142.17 101.6) (width 2.723) (layer "F.Cu") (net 2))
 (segment (start 147.25 100.076) (end 150.044 100.076) (width 0.508) (layer "F.Cu") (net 3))
 (segment (start 145.98 104.394) (end 147.25 103.124) (width 0.508) (layer "F.Cu") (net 3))
 (segment (start 147.25 103.124) (end 150.044 103.124) (width 0.508) (layer "F.Cu") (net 3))
 (segment (start 145.98 98.806) (end 147.25 100.076) (width 0.508) (layer "F.Cu") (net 3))
 (via (at 145.034 104.648) (size 0.8) (drill 0.5) (layers "F.Cu" "B.Cu") (free) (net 3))
 (via (at 143.764 98.552) (size 0.8) (drill 0.5) (layers "F.Cu" "B.Cu") (free) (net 3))
 (via (at 141.097 107.188) (size 0.8) (drill 0.5) (layers "F.Cu" "B.Cu") (free) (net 3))
 (via (at 146.488 98.806) (size 0.8) (drill 0.5) (layers "F.Cu" "B.Cu") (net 3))
 (via (at 144.78 98.552) (size 0.8) (drill 0.5) (layers "F.Cu" "B.Cu") (free) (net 3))
 (via (at 146.488 104.394) (size 0.8) (drill 0.5) (layers "F.Cu" "B.Cu") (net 3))
 (via (at 143.637 104.648) (size 0.8) (drill 0.5) (layers "F.Cu" "B.Cu") (free) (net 3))
 (via (at 142.748 98.044) (size 0.8) (drill 0.5) (layers "F.Cu" "B.Cu") (free) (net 3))
 (via (at 142.367 105.918) (size 0.8) (drill 0.5) (layers "F.Cu" "B.Cu") (free) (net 3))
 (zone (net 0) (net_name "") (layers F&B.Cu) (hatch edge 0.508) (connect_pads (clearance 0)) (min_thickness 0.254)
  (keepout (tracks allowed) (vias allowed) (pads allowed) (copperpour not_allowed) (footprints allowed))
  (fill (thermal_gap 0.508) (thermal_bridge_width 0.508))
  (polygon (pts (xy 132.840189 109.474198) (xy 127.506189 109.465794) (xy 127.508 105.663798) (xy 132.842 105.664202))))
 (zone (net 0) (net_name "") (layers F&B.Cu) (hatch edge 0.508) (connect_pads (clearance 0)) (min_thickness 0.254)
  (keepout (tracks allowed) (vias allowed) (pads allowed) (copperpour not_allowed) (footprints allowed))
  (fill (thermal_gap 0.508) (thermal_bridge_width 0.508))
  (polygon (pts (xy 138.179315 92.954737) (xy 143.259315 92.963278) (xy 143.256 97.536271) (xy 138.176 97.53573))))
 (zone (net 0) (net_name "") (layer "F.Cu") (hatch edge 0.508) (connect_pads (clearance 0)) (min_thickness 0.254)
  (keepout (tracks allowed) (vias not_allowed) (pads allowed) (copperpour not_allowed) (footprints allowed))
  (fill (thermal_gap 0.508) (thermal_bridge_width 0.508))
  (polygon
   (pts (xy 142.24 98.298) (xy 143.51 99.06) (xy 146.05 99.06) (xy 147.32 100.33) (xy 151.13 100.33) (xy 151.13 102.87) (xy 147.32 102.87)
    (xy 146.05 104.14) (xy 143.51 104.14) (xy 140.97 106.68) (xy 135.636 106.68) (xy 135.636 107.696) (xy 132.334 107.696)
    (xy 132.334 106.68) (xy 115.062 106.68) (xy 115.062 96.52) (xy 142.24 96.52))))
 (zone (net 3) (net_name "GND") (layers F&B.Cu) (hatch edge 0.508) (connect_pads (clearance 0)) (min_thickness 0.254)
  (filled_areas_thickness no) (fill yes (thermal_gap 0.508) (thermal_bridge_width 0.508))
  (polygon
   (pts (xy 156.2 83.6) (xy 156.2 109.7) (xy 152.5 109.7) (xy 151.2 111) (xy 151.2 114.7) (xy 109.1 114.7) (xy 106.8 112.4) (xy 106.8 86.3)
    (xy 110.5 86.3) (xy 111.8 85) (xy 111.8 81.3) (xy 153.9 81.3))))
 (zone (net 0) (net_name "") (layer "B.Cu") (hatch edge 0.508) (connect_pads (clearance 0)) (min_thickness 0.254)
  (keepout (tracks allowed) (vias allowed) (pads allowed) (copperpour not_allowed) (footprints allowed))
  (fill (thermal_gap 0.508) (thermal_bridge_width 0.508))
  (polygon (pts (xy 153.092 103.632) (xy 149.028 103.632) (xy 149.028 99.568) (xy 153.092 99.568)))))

